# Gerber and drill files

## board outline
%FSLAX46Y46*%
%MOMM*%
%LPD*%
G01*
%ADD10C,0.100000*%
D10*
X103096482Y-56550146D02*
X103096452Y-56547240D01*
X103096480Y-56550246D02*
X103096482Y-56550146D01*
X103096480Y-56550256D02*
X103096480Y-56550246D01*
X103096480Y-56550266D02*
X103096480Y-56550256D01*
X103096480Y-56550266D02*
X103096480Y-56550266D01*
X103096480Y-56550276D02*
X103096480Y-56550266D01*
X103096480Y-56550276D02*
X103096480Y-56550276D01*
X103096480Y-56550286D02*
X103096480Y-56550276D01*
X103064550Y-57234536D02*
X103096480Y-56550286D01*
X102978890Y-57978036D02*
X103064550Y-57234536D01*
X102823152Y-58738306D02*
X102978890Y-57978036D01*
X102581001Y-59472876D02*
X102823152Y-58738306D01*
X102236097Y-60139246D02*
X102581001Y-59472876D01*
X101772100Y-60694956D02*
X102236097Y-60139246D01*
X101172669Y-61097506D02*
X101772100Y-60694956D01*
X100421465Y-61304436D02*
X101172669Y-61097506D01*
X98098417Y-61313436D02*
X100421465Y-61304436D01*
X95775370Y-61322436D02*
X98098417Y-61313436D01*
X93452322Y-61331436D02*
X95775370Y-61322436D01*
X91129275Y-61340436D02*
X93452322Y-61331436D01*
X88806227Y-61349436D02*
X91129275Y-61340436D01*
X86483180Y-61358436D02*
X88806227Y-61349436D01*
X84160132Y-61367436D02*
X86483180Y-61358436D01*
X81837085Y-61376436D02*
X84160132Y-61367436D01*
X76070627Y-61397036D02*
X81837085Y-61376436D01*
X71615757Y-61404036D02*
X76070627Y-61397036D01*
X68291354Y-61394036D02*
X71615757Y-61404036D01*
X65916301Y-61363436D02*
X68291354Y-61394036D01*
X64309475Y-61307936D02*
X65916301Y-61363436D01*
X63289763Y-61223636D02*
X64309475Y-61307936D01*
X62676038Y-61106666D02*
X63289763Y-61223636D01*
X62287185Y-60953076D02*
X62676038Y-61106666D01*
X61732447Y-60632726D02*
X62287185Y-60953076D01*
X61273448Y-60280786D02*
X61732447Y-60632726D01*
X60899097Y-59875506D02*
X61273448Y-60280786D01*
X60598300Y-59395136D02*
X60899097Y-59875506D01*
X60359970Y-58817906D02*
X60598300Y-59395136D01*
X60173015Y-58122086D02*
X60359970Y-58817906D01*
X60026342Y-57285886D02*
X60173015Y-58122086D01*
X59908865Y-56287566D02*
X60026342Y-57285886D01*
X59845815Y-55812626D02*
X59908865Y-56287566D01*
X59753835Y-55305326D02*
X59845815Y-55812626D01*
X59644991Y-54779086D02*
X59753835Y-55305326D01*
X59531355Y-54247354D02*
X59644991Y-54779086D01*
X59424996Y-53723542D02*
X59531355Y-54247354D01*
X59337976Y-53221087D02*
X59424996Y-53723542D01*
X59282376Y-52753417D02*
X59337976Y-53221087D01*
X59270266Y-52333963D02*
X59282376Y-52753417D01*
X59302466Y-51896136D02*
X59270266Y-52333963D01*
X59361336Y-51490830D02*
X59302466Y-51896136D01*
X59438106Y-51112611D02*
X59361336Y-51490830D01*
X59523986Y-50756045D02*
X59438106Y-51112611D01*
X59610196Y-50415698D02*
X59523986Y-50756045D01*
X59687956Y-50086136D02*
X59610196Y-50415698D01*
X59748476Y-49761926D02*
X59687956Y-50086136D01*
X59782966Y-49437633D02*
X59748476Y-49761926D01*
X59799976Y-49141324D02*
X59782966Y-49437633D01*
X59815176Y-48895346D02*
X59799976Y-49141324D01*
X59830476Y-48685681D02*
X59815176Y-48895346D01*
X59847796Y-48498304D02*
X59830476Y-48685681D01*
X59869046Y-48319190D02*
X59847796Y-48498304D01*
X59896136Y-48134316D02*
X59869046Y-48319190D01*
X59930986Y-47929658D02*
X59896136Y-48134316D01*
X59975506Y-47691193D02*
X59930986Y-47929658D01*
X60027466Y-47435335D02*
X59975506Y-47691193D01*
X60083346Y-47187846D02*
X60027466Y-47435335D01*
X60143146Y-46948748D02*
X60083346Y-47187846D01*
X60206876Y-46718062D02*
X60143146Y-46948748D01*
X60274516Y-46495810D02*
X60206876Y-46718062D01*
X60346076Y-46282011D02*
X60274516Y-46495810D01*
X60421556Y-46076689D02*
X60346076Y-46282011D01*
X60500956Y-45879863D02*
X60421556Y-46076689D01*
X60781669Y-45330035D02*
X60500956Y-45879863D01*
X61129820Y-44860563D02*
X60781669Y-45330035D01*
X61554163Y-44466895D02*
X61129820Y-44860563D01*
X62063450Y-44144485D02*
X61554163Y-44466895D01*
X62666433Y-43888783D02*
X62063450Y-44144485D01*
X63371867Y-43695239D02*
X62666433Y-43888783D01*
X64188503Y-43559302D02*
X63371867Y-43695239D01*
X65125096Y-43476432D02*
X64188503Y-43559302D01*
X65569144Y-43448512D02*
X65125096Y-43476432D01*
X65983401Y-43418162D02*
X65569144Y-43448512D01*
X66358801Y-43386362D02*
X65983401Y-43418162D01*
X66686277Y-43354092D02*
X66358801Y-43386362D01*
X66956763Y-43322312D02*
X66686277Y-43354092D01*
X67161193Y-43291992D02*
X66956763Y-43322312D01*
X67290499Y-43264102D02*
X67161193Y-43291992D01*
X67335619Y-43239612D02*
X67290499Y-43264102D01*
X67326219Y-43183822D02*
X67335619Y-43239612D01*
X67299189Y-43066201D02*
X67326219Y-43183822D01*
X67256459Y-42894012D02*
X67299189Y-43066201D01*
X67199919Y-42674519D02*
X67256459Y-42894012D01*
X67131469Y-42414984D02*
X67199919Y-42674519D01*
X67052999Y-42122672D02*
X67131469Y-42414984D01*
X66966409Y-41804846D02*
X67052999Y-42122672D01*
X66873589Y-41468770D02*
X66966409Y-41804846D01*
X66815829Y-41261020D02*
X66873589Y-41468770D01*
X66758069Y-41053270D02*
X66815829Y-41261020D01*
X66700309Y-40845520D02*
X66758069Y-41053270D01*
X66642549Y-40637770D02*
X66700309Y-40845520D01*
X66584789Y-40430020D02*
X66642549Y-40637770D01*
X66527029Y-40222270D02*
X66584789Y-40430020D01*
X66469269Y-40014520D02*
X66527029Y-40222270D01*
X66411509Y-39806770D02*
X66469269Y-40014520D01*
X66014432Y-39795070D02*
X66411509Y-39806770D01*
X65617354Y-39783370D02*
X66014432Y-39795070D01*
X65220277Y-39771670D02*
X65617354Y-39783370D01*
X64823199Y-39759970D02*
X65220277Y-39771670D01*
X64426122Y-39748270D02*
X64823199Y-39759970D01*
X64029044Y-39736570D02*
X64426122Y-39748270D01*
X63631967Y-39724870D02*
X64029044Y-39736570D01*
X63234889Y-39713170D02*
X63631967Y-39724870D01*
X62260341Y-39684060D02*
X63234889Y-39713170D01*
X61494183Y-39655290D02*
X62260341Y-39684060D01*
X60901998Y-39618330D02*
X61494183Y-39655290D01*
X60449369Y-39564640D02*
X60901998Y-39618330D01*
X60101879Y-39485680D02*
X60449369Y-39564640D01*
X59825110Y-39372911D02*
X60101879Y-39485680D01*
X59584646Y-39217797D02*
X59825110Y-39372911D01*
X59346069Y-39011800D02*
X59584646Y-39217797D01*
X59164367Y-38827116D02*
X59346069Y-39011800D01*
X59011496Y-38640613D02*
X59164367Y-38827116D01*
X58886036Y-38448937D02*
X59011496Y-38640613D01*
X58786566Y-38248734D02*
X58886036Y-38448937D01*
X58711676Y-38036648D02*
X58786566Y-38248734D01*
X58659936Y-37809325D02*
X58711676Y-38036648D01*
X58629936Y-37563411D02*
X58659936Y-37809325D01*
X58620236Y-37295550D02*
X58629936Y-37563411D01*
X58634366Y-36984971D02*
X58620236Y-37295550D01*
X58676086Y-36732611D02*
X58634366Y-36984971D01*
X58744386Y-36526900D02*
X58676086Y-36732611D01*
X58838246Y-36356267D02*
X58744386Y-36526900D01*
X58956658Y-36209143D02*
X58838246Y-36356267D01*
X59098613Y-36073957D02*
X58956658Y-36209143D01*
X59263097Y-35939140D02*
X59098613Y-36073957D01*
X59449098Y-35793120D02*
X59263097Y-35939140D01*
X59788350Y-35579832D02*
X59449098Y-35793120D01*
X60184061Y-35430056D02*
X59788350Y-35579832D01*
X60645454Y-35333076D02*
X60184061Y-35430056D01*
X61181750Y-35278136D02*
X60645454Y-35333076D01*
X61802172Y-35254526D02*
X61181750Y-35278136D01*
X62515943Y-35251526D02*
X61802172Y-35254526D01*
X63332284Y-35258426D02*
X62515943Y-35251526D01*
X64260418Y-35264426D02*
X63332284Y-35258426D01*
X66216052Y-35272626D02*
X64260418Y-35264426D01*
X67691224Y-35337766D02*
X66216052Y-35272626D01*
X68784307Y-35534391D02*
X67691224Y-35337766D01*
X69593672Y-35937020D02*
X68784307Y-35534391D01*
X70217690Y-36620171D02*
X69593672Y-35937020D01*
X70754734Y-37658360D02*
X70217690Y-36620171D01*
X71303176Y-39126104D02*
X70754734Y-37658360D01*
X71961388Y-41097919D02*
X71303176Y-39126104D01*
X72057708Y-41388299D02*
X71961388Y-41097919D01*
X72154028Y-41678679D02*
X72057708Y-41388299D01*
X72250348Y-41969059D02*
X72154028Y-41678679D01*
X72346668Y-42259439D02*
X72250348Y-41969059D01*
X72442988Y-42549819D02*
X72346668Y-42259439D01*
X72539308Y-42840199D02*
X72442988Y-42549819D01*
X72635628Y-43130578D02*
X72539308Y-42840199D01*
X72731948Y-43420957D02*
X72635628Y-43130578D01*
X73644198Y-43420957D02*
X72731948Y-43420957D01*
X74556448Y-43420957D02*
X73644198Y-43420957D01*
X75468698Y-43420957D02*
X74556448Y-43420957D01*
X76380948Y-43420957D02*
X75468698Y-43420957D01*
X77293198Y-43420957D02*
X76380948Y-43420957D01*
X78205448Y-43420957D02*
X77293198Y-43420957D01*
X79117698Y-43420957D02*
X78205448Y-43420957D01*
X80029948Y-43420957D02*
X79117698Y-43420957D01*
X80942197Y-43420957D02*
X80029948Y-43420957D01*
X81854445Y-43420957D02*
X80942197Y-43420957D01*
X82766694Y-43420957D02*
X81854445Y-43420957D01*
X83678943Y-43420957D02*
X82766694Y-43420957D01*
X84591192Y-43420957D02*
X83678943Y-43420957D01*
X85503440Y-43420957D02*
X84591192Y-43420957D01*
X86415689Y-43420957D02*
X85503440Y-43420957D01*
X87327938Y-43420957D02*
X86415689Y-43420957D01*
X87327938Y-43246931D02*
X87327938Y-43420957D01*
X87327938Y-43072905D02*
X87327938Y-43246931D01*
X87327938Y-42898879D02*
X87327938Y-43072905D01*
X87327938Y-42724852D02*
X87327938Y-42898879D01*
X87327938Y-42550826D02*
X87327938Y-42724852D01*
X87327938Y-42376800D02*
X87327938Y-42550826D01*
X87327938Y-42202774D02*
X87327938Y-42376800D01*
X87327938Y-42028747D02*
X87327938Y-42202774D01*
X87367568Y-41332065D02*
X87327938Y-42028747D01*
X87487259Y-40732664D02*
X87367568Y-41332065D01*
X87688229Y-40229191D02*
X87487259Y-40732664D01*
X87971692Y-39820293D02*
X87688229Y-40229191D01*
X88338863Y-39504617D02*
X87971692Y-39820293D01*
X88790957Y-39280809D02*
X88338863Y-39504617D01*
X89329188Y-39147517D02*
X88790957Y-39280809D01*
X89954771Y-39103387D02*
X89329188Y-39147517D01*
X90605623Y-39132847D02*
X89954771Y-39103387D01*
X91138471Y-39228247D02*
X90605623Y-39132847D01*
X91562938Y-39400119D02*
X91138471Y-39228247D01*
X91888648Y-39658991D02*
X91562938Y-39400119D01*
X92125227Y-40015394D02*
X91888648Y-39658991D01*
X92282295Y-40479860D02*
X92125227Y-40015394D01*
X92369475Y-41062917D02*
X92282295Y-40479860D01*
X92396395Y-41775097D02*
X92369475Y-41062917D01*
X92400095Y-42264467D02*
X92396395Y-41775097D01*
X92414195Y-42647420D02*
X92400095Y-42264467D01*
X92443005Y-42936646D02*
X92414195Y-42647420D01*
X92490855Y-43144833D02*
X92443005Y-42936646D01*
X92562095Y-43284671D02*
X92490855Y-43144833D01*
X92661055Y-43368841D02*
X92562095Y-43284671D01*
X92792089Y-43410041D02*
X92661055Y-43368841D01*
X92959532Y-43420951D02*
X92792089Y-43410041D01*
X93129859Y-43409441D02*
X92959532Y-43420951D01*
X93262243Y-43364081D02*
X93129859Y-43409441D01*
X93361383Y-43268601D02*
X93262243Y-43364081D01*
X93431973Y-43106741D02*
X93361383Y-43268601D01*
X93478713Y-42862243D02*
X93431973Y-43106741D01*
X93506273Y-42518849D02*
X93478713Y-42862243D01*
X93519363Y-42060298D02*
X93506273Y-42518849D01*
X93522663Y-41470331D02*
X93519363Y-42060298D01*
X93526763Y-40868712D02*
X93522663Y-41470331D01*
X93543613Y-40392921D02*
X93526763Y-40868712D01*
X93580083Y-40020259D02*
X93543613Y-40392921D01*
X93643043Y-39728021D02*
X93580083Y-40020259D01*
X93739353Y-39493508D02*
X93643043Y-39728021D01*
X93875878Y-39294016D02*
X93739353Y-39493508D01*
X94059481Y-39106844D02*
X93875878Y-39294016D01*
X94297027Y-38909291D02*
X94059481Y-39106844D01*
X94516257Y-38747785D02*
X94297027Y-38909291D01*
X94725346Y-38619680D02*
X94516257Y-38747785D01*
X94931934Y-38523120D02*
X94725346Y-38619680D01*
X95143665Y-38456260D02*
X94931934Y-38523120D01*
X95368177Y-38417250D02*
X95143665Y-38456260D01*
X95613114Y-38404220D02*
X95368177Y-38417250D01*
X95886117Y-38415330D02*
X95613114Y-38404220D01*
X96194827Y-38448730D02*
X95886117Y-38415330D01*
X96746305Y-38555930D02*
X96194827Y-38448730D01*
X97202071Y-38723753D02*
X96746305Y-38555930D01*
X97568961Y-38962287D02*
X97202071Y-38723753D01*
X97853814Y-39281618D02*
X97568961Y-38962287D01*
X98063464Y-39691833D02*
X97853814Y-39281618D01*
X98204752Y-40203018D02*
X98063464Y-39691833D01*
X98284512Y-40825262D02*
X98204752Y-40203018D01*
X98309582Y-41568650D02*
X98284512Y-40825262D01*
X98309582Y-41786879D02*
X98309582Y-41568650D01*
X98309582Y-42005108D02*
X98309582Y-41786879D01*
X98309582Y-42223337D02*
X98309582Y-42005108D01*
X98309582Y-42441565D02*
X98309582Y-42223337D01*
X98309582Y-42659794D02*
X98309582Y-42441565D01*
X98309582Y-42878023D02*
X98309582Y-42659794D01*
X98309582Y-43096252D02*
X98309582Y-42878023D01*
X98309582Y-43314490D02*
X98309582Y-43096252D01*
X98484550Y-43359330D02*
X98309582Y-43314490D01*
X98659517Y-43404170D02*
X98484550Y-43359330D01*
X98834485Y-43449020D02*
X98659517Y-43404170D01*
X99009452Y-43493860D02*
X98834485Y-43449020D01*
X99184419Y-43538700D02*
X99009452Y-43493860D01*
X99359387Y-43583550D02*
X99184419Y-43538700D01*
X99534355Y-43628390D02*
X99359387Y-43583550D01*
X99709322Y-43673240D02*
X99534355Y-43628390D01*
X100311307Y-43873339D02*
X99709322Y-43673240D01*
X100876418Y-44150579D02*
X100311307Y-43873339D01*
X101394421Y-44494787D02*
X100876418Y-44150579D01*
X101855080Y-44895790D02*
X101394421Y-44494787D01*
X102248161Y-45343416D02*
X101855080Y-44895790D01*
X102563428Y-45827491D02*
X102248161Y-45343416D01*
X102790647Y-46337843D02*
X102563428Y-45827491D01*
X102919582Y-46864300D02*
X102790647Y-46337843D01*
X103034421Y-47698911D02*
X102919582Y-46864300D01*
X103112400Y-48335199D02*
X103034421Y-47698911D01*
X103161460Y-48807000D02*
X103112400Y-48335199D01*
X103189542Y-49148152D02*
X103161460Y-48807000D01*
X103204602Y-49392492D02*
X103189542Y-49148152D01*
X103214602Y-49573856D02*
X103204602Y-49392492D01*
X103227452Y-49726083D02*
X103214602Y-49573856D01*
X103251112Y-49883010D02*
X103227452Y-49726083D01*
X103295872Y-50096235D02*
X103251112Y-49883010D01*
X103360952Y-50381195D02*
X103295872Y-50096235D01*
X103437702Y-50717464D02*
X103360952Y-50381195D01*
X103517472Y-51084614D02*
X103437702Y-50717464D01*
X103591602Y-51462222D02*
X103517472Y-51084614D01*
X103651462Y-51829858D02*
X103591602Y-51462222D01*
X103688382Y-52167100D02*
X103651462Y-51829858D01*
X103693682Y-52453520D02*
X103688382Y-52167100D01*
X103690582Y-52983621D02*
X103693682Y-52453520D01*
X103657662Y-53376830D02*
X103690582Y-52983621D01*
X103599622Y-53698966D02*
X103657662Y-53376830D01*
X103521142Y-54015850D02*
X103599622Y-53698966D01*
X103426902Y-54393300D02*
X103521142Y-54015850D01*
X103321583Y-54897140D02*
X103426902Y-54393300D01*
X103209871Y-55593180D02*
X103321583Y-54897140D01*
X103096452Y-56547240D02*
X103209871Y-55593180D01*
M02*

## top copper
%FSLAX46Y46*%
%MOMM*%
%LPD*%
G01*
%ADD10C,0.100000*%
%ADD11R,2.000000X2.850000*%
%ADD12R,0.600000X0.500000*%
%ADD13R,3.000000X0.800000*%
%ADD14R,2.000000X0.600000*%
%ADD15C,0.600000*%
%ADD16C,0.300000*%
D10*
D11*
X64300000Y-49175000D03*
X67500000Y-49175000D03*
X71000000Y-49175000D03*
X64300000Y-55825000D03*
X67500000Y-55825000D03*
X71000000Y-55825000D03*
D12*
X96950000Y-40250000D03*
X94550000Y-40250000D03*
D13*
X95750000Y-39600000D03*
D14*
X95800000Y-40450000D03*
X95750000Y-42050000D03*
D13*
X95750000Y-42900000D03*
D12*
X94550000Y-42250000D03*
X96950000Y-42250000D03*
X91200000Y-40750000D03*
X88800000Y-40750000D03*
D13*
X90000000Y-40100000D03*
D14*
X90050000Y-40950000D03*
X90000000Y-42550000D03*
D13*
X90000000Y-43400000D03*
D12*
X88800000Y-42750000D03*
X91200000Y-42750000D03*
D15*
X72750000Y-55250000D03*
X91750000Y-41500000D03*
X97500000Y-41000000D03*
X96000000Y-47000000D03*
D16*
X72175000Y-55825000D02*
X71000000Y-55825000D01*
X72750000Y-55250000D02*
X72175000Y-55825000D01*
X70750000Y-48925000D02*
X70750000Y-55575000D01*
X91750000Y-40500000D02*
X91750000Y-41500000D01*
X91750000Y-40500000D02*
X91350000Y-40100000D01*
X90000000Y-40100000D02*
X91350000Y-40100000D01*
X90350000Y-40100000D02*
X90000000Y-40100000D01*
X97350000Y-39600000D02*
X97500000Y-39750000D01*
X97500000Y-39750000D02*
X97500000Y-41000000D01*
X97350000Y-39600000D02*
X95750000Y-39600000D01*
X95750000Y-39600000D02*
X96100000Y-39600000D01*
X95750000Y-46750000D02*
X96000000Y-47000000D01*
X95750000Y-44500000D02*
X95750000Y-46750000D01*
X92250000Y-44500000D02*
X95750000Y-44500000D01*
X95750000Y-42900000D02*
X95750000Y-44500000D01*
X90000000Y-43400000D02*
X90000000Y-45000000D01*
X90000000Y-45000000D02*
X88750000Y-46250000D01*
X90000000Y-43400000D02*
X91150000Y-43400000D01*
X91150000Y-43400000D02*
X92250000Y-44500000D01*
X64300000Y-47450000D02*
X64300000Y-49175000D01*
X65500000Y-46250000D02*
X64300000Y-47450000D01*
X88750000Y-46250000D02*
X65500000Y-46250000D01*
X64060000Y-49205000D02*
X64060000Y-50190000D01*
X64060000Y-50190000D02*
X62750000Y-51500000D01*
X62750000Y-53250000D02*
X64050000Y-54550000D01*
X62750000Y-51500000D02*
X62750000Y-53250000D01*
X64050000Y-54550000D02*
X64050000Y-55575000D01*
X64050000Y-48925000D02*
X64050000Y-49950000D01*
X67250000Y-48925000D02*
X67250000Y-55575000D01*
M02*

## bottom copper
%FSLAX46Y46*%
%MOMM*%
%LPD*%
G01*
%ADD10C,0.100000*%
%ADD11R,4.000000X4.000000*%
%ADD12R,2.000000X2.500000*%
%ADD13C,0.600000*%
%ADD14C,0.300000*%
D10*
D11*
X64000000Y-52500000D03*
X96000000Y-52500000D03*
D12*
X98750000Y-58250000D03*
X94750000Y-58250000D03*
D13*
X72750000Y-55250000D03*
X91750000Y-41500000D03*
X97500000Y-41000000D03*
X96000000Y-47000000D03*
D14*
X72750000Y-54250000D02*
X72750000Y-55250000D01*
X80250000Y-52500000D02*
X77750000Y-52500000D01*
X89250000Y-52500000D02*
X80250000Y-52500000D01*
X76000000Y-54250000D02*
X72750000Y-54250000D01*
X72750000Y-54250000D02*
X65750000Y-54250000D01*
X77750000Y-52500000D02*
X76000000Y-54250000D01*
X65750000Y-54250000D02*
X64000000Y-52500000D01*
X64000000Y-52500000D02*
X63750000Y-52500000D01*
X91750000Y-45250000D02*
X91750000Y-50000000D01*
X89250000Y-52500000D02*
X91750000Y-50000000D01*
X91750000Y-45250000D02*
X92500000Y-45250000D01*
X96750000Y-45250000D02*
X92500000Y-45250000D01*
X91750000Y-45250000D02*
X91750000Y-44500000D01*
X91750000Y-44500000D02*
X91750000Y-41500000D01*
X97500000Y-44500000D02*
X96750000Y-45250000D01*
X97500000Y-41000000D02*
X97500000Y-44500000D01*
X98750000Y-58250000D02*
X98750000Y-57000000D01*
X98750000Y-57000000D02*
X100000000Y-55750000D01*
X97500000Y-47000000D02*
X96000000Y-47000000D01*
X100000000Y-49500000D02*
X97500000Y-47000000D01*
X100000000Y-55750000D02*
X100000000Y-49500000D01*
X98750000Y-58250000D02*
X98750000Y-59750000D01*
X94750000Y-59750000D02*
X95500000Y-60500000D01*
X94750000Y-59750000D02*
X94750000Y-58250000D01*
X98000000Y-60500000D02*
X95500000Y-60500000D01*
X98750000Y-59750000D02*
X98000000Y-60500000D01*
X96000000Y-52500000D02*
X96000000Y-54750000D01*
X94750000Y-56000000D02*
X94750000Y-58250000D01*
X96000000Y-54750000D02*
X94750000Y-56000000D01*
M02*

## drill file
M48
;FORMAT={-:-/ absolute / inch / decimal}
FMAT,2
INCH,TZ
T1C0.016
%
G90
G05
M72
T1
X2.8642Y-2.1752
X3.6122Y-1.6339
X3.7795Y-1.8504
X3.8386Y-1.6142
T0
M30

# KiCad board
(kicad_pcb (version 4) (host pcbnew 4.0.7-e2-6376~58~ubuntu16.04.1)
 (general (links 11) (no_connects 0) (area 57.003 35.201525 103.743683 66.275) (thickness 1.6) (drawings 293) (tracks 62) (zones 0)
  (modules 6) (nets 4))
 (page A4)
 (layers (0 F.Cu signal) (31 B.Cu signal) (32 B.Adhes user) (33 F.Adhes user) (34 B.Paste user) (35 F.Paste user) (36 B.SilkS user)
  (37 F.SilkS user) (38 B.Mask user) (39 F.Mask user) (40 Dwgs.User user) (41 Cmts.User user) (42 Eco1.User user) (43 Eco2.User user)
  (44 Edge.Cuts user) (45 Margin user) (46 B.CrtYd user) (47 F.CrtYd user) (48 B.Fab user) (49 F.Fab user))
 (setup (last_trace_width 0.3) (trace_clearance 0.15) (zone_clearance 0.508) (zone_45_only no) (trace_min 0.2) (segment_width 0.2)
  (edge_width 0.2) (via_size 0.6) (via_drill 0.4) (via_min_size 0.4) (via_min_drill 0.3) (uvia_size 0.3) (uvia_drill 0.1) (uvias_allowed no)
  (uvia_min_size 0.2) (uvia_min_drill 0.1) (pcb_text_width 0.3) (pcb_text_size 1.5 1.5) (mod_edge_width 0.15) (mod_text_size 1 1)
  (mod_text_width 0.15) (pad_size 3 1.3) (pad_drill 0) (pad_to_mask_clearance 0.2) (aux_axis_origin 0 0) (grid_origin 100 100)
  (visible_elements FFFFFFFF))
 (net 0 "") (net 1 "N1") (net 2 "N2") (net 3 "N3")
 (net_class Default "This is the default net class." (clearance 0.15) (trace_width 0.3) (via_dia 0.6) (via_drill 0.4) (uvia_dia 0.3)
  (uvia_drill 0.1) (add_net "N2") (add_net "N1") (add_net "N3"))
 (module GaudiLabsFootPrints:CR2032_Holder (layer B.Cu) (at 80 52.5)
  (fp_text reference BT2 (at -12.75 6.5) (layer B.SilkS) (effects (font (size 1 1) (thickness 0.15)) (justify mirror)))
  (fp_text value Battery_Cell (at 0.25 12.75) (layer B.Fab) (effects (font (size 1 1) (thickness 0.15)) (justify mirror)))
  (pad 2 smd rect (at -16 0) (size 4 4) (layers B.Cu B.Paste B.Mask) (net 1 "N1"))
  (pad 1 smd rect (at 16 0) (size 4 4) (layers B.Cu B.Paste B.Mask) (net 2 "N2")))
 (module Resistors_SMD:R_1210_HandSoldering (layer B.Cu) (at 96.75 58.25 180)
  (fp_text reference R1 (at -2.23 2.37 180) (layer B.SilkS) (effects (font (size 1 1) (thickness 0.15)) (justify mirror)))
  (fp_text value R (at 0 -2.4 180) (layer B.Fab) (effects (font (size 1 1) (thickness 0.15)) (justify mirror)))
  (pad 1 smd rect (at -2 0 180) (size 2 2.5) (layers B.Cu B.Paste B.Mask) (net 2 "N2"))
  (pad 2 smd rect (at 2 0 180) (size 2 2.5) (layers B.Cu B.Paste B.Mask) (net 2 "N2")))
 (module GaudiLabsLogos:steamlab (layer F.Cu) (at 81.14 48.34)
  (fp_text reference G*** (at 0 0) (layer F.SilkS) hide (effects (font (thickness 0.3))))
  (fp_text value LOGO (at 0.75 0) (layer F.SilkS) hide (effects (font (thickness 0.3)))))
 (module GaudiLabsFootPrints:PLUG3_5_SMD (layer F.Cu) (at 62.5 52.5 90)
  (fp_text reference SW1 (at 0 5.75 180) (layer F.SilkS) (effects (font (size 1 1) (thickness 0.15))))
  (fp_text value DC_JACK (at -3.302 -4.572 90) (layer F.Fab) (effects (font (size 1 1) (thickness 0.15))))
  (pad 1 smd rect (at 3.325 1.8 90) (size 2.85 2) (layers F.Cu F.Paste F.Mask) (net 2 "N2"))
  (pad 2 smd rect (at 3.325 5 90) (size 2.85 2) (layers F.Cu F.Paste F.Mask) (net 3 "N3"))
  (pad 3 smd rect (at 3.325 8.5 90) (size 2.85 2) (layers F.Cu F.Paste F.Mask) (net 1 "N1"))
  (pad 1 smd rect (at -3.325 1.8 90) (size 2.85 2) (layers F.Cu F.Paste F.Mask) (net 2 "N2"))
  (pad 2 smd rect (at -3.325 5 90) (size 2.85 2) (layers F.Cu F.Paste F.Mask) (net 3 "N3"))
  (pad 3 smd rect (at -3.325 8.5 90) (size 2.85 2) (layers F.Cu F.Paste F.Mask) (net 1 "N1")))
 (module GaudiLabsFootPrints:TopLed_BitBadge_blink (layer F.Cu) (at 95.75 41.25 180)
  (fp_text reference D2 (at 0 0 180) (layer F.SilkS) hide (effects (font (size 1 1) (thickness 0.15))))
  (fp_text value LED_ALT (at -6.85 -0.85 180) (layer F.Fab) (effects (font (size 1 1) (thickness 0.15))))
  (pad "" smd rect (at -1.2 1 180) (size 0.6 0.5) (layers F.Cu F.Paste F.Mask))
  (pad "" smd rect (at 1.2 1 180) (size 0.6 0.5) (layers F.Cu F.Paste F.Mask))
  (pad 1 smd rect (at 0 1.65 180) (size 3 0.8) (layers F.Cu F.Paste F.Mask) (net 1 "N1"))
  (pad "" smd rect (at -0.05 0.8 180) (size 2 0.6) (layers F.Cu F.Paste F.Mask))
  (pad "" smd rect (at 0 -0.8 180) (size 2 0.6) (layers F.Cu F.Paste F.Mask))
  (pad 2 smd rect (at 0 -1.65 180) (size 3 0.8) (layers F.Cu F.Paste F.Mask) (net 2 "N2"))
  (pad "" smd rect (at 1.2 -1 180) (size 0.6 0.5) (layers F.Cu F.Paste F.Mask))
  (pad "" smd rect (at -1.2 -1 180) (size 0.6 0.5) (layers F.Cu F.Paste F.Mask)))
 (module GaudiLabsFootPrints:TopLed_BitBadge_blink (layer F.Cu) (at 90 41.75 180)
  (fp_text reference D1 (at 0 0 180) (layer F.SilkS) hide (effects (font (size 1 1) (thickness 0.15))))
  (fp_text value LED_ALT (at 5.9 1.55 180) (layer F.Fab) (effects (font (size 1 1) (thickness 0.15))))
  (pad "" smd rect (at -1.2 1 180) (size 0.6 0.5) (layers F.Cu F.Paste F.Mask))
  (pad "" smd rect (at 1.2 1 180) (size 0.6 0.5) (layers F.Cu F.Paste F.Mask))
  (pad 1 smd rect (at 0 1.65 180) (size 3 0.8) (layers F.Cu F.Paste F.Mask) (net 1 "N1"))
  (pad "" smd rect (at -0.05 0.8 180) (size 2 0.6) (layers F.Cu F.Paste F.Mask))
  (pad "" smd rect (at 0 -0.8 180) (size 2 0.6) (layers F.Cu F.Paste F.Mask))
  (pad 2 smd rect (at 0 -1.65 180) (size 3 0.8) (layers F.Cu F.Paste F.Mask) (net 2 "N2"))
  (pad "" smd rect (at 1.2 -1 180) (size 0.6 0.5) (layers F.Cu F.Paste F.Mask))
  (pad "" smd rect (at -1.2 -1 180) (size 0.6 0.5) (layers F.Cu F.Paste F.Mask)))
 (gr_line (start 103.096482 56.550146) (end 103.096452 56.54724) (layer Edge.Cuts) (width 0.1))
 (gr_line (start 103.09648 56.550246) (end 103.096482 56.550146) (layer Edge.Cuts) (width 0.1))
 (gr_line (start 103.09648 56.550256) (end 103.09648 56.550246) (layer Edge.Cuts) (width 0.1))
 (gr_line (start 103.09648 56.550266) (end 103.09648 56.550256) (layer Edge.Cuts) (width 0.1))
 (gr_line (start 103.09648 56.550266) (end 103.09648 56.550266) (layer Edge.Cuts) (width 0.1))
 (gr_line (start 103.09648 56.550276) (end 103.09648 56.550266) (layer Edge.Cuts) (width 0.1))
 (gr_line (start 103.09648 56.550276) (end 103.09648 56.550276) (layer Edge.Cuts) (width 0.1))
 (gr_line (start 103.09648 56.550286) (end 103.09648 56.550276) (layer Edge.Cuts) (width 0.1))
 (gr_line (start 103.06455 57.234536) (end 103.09648 56.550286) (layer Edge.Cuts) (width 0.1))
 (gr_line (start 102.97889 57.978036) (end 103.06455 57.234536) (layer Edge.Cuts) (width 0.1))
 (gr_line (start 102.823152 58.738306) (end 102.97889 57.978036) (layer Edge.Cuts) (width 0.1))
 (gr_line (start 102.581001 59.472876) (end 102.823152 58.738306) (layer Edge.Cuts) (width 0.1))
 (gr_line (start 102.236097 60.139246) (end 102.581001 59.472876) (layer Edge.Cuts) (width 0.1))
 (gr_line (start 101.7721 60.694956) (end 102.236097 60.139246) (layer Edge.Cuts) (width 0.1))
 (gr_line (start 101.172669 61.097506) (end 101.7721 60.694956) (layer Edge.Cuts) (width 0.1))
 (gr_line (start 100.421465 61.304436) (end 101.172669 61.097506) (layer Edge.Cuts) (width 0.1))
 (gr_line (start 98.098417 61.313436) (end 100.421465 61.304436) (layer Edge.Cuts) (width 0.1))
 (gr_line (start 95.77537 61.322436) (end 98.098417 61.313436) (layer Edge.Cuts) (width 0.1))
 (gr_line (start 93.452322 61.331436) (end 95.77537 61.322436) (layer Edge.Cuts) (width 0.1))
 (gr_line (start 91.129275 61.340436) (end 93.452322 61.331436) (layer Edge.Cuts) (width 0.1))
 (gr_line (start 88.806227 61.349436) (end 91.129275 61.340436) (layer Edge.Cuts) (width 0.1))
 (gr_line (start 86.48318 61.358436) (end 88.806227 61.349436) (layer Edge.Cuts) (width 0.1))
 (gr_line (start 84.160132 61.367436) (end 86.48318 61.358436) (layer Edge.Cuts) (width 0.1))
 (gr_line (start 81.837085 61.376436) (end 84.160132 61.367436) (layer Edge.Cuts) (width 0.1))
 (gr_line (start 76.070627 61.397036) (end 81.837085 61.376436) (layer Edge.Cuts) (width 0.1))
 (gr_line (start 71.615757 61.404036) (end 76.070627 61.397036) (layer Edge.Cuts) (width 0.1))
 (gr_line (start 68.291354 61.394036) (end 71.615757 61.404036) (layer Edge.Cuts) (width 0.1))
 (gr_line (start 65.916301 61.363436) (end 68.291354 61.394036) (layer Edge.Cuts) (width 0.1))
 (gr_line (start 64.309475 61.307936) (end 65.916301 61.363436) (layer Edge.Cuts) (width 0.1))
 (gr_line (start 63.289763 61.223636) (end 64.309475 61.307936) (layer Edge.Cuts) (width 0.1))
 (gr_line (start 62.676038 61.106666) (end 63.289763 61.223636) (layer Edge.Cuts) (width 0.1))
 (gr_line (start 62.287185 60.953076) (end 62.676038 61.106666) (layer Edge.Cuts) (width 0.1))
 (gr_line (start 61.732447 60.632726) (end 62.287185 60.953076) (layer Edge.Cuts) (width 0.1))
 (gr_line (start 61.273448 60.280786) (end 61.732447 60.632726) (layer Edge.Cuts) (width 0.1))
 (gr_line (start 60.899097 59.875506) (end 61.273448 60.280786) (layer Edge.Cuts) (width 0.1))
 (gr_line (start 60.5983 59.395136) (end 60.899097 59.875506) (layer Edge.Cuts) (width 0.1))
 (gr_line (start 60.35997 58.817906) (end 60.5983 59.395136) (layer Edge.Cuts) (width 0.1))
 (gr_line (start 60.173015 58.122086) (end 60.35997 58.817906) (layer Edge.Cuts) (width 0.1))
 (gr_line (start 60.026342 57.285886) (end 60.173015 58.122086) (layer Edge.Cuts) (width 0.1))
 (gr_line (start 59.908865 56.287566) (end 60.026342 57.285886) (layer Edge.Cuts) (width 0.1))
 (gr_line (start 59.845815 55.812626) (end 59.908865 56.287566) (layer Edge.Cuts) (width 0.1))
 (gr_line (start 59.753835 55.305326) (end 59.845815 55.812626) (layer Edge.Cuts) (width 0.1))
 (gr_line (start 59.644991 54.779086) (end 59.753835 55.305326) (layer Edge.Cuts) (width 0.1))
 (gr_line (start 59.531355 54.247354) (end 59.644991 54.779086) (layer Edge.Cuts) (width 0.1))
 (gr_line (start 59.424996 53.723542) (end 59.531355 54.247354) (layer Edge.Cuts) (width 0.1))
 (gr_line (start 59.337976 53.221087) (end 59.424996 53.723542) (layer Edge.Cuts) (width 0.1))
 (gr_line (start 59.282376 52.753417) (end 59.337976 53.221087) (layer Edge.Cuts) (width 0.1))
 (gr_line (start 59.270266 52.333963) (end 59.282376 52.753417) (layer Edge.Cuts) (width 0.1))
 (gr_line (start 59.302466 51.896136) (end 59.270266 52.333963) (layer Edge.Cuts) (width 0.1))
 (gr_line (start 59.361336 51.49083) (end 59.302466 51.896136) (layer Edge.Cuts) (width 0.1))
 (gr_line (start 59.438106 51.112611) (end 59.361336 51.49083) (layer Edge.Cuts) (width 0.1))
 (gr_line (start 59.523986 50.756045) (end 59.438106 51.112611) (layer Edge.Cuts) (width 0.1))
 (gr_line (start 59.610196 50.415698) (end 59.523986 50.756045) (layer Edge.Cuts) (width 0.1))
 (gr_line (start 59.687956 50.086136) (end 59.610196 50.415698) (layer Edge.Cuts) (width 0.1))
 (gr_line (start 59.748476 49.761926) (end 59.687956 50.086136) (layer Edge.Cuts) (width 0.1))
 (gr_line (start 59.782966 49.437633) (end 59.748476 49.761926) (layer Edge.Cuts) (width 0.1))
 (gr_line (start 59.799976 49.141324) (end 59.782966 49.437633) (layer Edge.Cuts) (width 0.1))
 (gr_line (start 59.815176 48.895346) (end 59.799976 49.141324) (layer Edge.Cuts) (width 0.1))
 (gr_line (start 59.830476 48.685681) (end 59.815176 48.895346) (layer Edge.Cuts) (width 0.1))
 (gr_line (start 59.847796 48.498304) (end 59.830476 48.685681) (layer Edge.Cuts) (width 0.1))
 (gr_line (start 59.869046 48.31919) (end 59.847796 48.498304) (layer Edge.Cuts) (width 0.1))
 (gr_line (start 59.896136 48.134316) (end 59.869046 48.31919) (layer Edge.Cuts) (width 0.1))
 (gr_line (start 59.930986 47.929658) (end 59.896136 48.134316) (layer Edge.Cuts) (width 0.1))
 (gr_line (start 59.975506 47.691193) (end 59.930986 47.929658) (layer Edge.Cuts) (width 0.1))
 (gr_line (start 60.027466 47.435335) (end 59.975506 47.691193) (layer Edge.Cuts) (width 0.1))
 (gr_line (start 60.083346 47.187846) (end 60.027466 47.435335) (layer Edge.Cuts) (width 0.1))
 (gr_line (start 60.143146 46.948748) (end 60.083346 47.187846) (layer Edge.Cuts) (width 0.1))
 (gr_line (start 60.206876 46.718062) (end 60.143146 46.948748) (layer Edge.Cuts) (width 0.1))
 (gr_line (start 60.274516 46.49581) (end 60.206876 46.718062) (layer Edge.Cuts) (width 0.1))
 (gr_line (start 60.346076 46.282011) (end 60.274516 46.49581) (layer Edge.Cuts) (width 0.1))
 (gr_line (start 60.421556 46.076689) (end 60.346076 46.282011) (layer Edge.Cuts) (width 0.1))
 (gr_line (start 60.500956 45.879863) (end 60.421556 46.076689) (layer Edge.Cuts) (width 0.1))
 (gr_line (start 60.781669 45.330035) (end 60.500956 45.879863) (layer Edge.Cuts) (width 0.1))
 (gr_line (start 61.12982 44.860563) (end 60.781669 45.330035) (layer Edge.Cuts) (width 0.1))
 (gr_line (start 61.554163 44.466895) (end 61.12982 44.860563) (layer Edge.Cuts) (width 0.1))
 (gr_line (start 62.06345 44.144485) (end 61.554163 44.466895) (layer Edge.Cuts) (width 0.1))
 (gr_line (start 62.666433 43.888783) (end 62.06345 44.144485) (layer Edge.Cuts) (width 0.1))
 (gr_line (start 63.371867 43.695239) (end 62.666433 43.888783) (layer Edge.Cuts) (width 0.1))
 (gr_line (start 64.188503 43.559302) (end 63.371867 43.695239) (layer Edge.Cuts) (width 0.1))
 (gr_line (start 65.125096 43.476432) (end 64.188503 43.559302) (layer Edge.Cuts) (width 0.1))
 (gr_line (start 65.569144 43.448512) (end 65.125096 43.476432) (layer Edge.Cuts) (width 0.1))
 (gr_line (start 65.983401 43.418162) (end 65.569144 43.448512) (layer Edge.Cuts) (width 0.1))
 (gr_line (start 66.358801 43.386362) (end 65.983401 43.418162) (layer Edge.Cuts) (width 0.1))
 (gr_line (start 66.686277 43.354092) (end 66.358801 43.386362) (layer Edge.Cuts) (width 0.1))
 (gr_line (start 66.956763 43.322312) (end 66.686277 43.354092) (layer Edge.Cuts) (width 0.1))
 (gr_line (start 67.161193 43.291992) (end 66.956763 43.322312) (layer Edge.Cuts) (width 0.1))
 (gr_line (start 67.290499 43.264102) (end 67.161193 43.291992) (layer Edge.Cuts) (width 0.1))
 (gr_line (start 67.335619 43.239612) (end 67.290499 43.264102) (layer Edge.Cuts) (width 0.1))
 (gr_line (start 67.326219 43.183822) (end 67.335619 43.239612) (layer Edge.Cuts) (width 0.1))
 (gr_line (start 67.299189 43.066201) (end 67.326219 43.183822) (layer Edge.Cuts) (width 0.1))
 (gr_line (start 67.256459 42.894012) (end 67.299189 43.066201) (layer Edge.Cuts) (width 0.1))
 (gr_line (start 67.199919 42.674519) (end 67.256459 42.894012) (layer Edge.Cuts) (width 0.1))
 (gr_line (start 67.131469 42.414984) (end 67.199919 42.674519) (layer Edge.Cuts) (width 0.1))
 (gr_line (start 67.052999 42.122672) (end 67.131469 42.414984) (layer Edge.Cuts) (width 0.1))
 (gr_line (start 66.966409 41.804846) (end 67.052999 42.122672) (layer Edge.Cuts) (width 0.1))
 (gr_line (start 66.873589 41.46877) (end 66.966409 41.804846) (layer Edge.Cuts) (width 0.1))
 (gr_line (start 66.815829 41.26102) (end 66.873589 41.46877) (layer Edge.Cuts) (width 0.1))
 (gr_line (start 66.758069 41.05327) (end 66.815829 41.26102) (layer Edge.Cuts) (width 0.1))
 (gr_line (start 66.700309 40.84552) (end 66.758069 41.05327) (layer Edge.Cuts) (width 0.1))
 (gr_line (start 66.642549 40.63777) (end 66.700309 40.84552) (layer Edge.Cuts) (width 0.1))
 (gr_line (start 66.584789 40.43002) (end 66.642549 40.63777) (layer Edge.Cuts) (width 0.1))
 (gr_line (start 66.527029 40.22227) (end 66.584789 40.43002) (layer Edge.Cuts) (width 0.1))
 (gr_line (start 66.469269 40.01452) (end 66.527029 40.22227) (layer Edge.Cuts) (width 0.1))
 (gr_line (start 66.411509 39.80677) (end 66.469269 40.01452) (layer Edge.Cuts) (width 0.1))
 (gr_line (start 66.014432 39.79507) (end 66.411509 39.80677) (layer Edge.Cuts) (width 0.1))
 (gr_line (start 65.617354 39.78337) (end 66.014432 39.79507) (layer Edge.Cuts) (width 0.1))
 (gr_line (start 65.220277 39.77167) (end 65.617354 39.78337) (layer Edge.Cuts) (width 0.1))
 (gr_line (start 64.823199 39.75997) (end 65.220277 39.77167) (layer Edge.Cuts) (width 0.1))
 (gr_line (start 64.426122 39.74827) (end 64.823199 39.75997) (layer Edge.Cuts) (width 0.1))
 (gr_line (start 64.029044 39.73657) (end 64.426122 39.74827) (layer Edge.Cuts) (width 0.1))
 (gr_line (start 63.631967 39.72487) (end 64.029044 39.73657) (layer Edge.Cuts) (width 0.1))
 (gr_line (start 63.234889 39.71317) (end 63.631967 39.72487) (layer Edge.Cuts) (width 0.1))
 (gr_line (start 62.260341 39.68406) (end 63.234889 39.71317) (layer Edge.Cuts) (width 0.1))
 (gr_line (start 61.494183 39.65529) (end 62.260341 39.68406) (layer Edge.Cuts) (width 0.1))
 (gr_line (start 60.901998 39.61833) (end 61.494183 39.65529) (layer Edge.Cuts) (width 0.1))
 (gr_line (start 60.449369 39.56464) (end 60.901998 39.61833) (layer Edge.Cuts) (width 0.1))
 (gr_line (start 60.101879 39.48568) (end 60.449369 39.56464) (layer Edge.Cuts) (width 0.1))
 (gr_line (start 59.82511 39.372911) (end 60.101879 39.48568) (layer Edge.Cuts) (width 0.1))
 (gr_line (start 59.584646 39.217797) (end 59.82511 39.372911) (layer Edge.Cuts) (width 0.1))
 (gr_line (start 59.346069 39.0118) (end 59.584646 39.217797) (layer Edge.Cuts) (width 0.1))
 (gr_line (start 59.164367 38.827116) (end 59.346069 39.0118) (layer Edge.Cuts) (width 0.1))
 (gr_line (start 59.011496 38.640613) (end 59.164367 38.827116) (layer Edge.Cuts) (width 0.1))
 (gr_line (start 58.886036 38.448937) (end 59.011496 38.640613) (layer Edge.Cuts) (width 0.1))
 (gr_line (start 58.786566 38.248734) (end 58.886036 38.448937) (layer Edge.Cuts) (width 0.1))
 (gr_line (start 58.711676 38.036648) (end 58.786566 38.248734) (layer Edge.Cuts) (width 0.1))
 (gr_line (start 58.659936 37.809325) (end 58.711676 38.036648) (layer Edge.Cuts) (width 0.1))
 (gr_line (start 58.629936 37.563411) (end 58.659936 37.809325) (layer Edge.Cuts) (width 0.1))
 (gr_line (start 58.620236 37.29555) (end 58.629936 37.563411) (layer Edge.Cuts) (width 0.1))
 (gr_line (start 58.634366 36.984971) (end 58.620236 37.29555) (layer Edge.Cuts) (width 0.1))
 (gr_line (start 58.676086 36.732611) (end 58.634366 36.984971) (layer Edge.Cuts) (width 0.1))
 (gr_line (start 58.744386 36.5269) (end 58.676086 36.732611) (layer Edge.Cuts) (width 0.1))
 (gr_line (start 58.838246 36.356267) (end 58.744386 36.5269) (layer Edge.Cuts) (width 0.1))
 (gr_line (start 58.956658 36.209143) (end 58.838246 36.356267) (layer Edge.Cuts) (width 0.1))
 (gr_line (start 59.098613 36.073957) (end 58.956658 36.209143) (layer Edge.Cuts) (width 0.1))
 (gr_line (start 59.263097 35.93914) (end 59.098613 36.073957) (layer Edge.Cuts) (width 0.1))
 (gr_line (start 59.449098 35.79312) (end 59.263097 35.93914) (layer Edge.Cuts) (width 0.1))
 (gr_line (start 59.78835 35.579832) (end 59.449098 35.79312) (layer Edge.Cuts) (width 0.1))
 (gr_line (start 60.184061 35.430056) (end 59.78835 35.579832) (layer Edge.Cuts) (width 0.1))
 (gr_line (start 60.645454 35.333076) (end 60.184061 35.430056) (layer Edge.Cuts) (width 0.1))
 (gr_line (start 61.18175 35.278136) (end 60.645454 35.333076) (layer Edge.Cuts) (width 0.1))
 (gr_line (start 61.802172 35.254526) (end 61.18175 35.278136) (layer Edge.Cuts) (width 0.1))
 (gr_line (start 62.515943 35.251526) (end 61.802172 35.254526) (layer Edge.Cuts) (width 0.1))
 (gr_line (start 63.332284 35.258426) (end 62.515943 35.251526) (layer Edge.Cuts) (width 0.1))
 (gr_line (start 64.260418 35.264426) (end 63.332284 35.258426) (layer Edge.Cuts) (width 0.1))
 (gr_line (start 66.216052 35.272626) (end 64.260418 35.264426) (layer Edge.Cuts) (width 0.1))
 (gr_line (start 67.691224 35.337766) (end 66.216052 35.272626) (layer Edge.Cuts) (width 0.1))
 (gr_line (start 68.784307 35.534391) (end 67.691224 35.337766) (layer Edge.Cuts) (width 0.1))
 (gr_line (start 69.593672 35.93702) (end 68.784307 35.534391) (layer Edge.Cuts) (width 0.1))
 (gr_line (start 70.21769 36.620171) (end 69.593672 35.93702) (layer Edge.Cuts) (width 0.1))
 (gr_line (start 70.754734 37.65836) (end 70.21769 36.620171) (layer Edge.Cuts) (width 0.1))
 (gr_line (start 71.303176 39.126104) (end 70.754734 37.65836) (layer Edge.Cuts) (width 0.1))
 (gr_line (start 71.961388 41.097919) (end 71.303176 39.126104) (layer Edge.Cuts) (width 0.1))
 (gr_line (start 72.057708 41.388299) (end 71.961388 41.097919) (layer Edge.Cuts) (width 0.1))
 (gr_line (start 72.154028 41.678679) (end 72.057708 41.388299) (layer Edge.Cuts) (width 0.1))
 (gr_line (start 72.250348 41.969059) (end 72.154028 41.678679) (layer Edge.Cuts) (width 0.1))
 (gr_line (start 72.346668 42.259439) (end 72.250348 41.969059) (layer Edge.Cuts) (width 0.1))
 (gr_line (start 72.442988 42.549819) (end 72.346668 42.259439) (layer Edge.Cuts) (width 0.1))
 (gr_line (start 72.539308 42.840199) (end 72.442988 42.549819) (layer Edge.Cuts) (width 0.1))
 (gr_line (start 72.635628 43.130578) (end 72.539308 42.840199) (layer Edge.Cuts) (width 0.1))
 (gr_line (start 72.731948 43.420957) (end 72.635628 43.130578) (layer Edge.Cuts) (width 0.1))
 (gr_line (start 73.644198 43.420957) (end 72.731948 43.420957) (layer Edge.Cuts) (width 0.1))
 (gr_line (start 74.556448 43.420957) (end 73.644198 43.420957) (layer Edge.Cuts) (width 0.1))
 (gr_line (start 75.468698 43.420957) (end 74.556448 43.420957) (layer Edge.Cuts) (width 0.1))
 (gr_line (start 76.380948 43.420957) (end 75.468698 43.420957) (layer Edge.Cuts) (width 0.1))
 (gr_line (start 77.293198 43.420957) (end 76.380948 43.420957) (layer Edge.Cuts) (width 0.1))
 (gr_line (start 78.205448 43.420957) (end 77.293198 43.420957) (layer Edge.Cuts) (width 0.1))
 (gr_line (start 79.117698 43.420957) (end 78.205448 43.420957) (layer Edge.Cuts) (width 0.1))
 (gr_line (start 80.029948 43.420957) (end 79.117698 43.420957) (layer Edge.Cuts) (width 0.1))
 (gr_line (start 80.942197 43.420957) (end 80.029948 43.420957) (layer Edge.Cuts) (width 0.1))
 (gr_line (start 81.854445 43.420957) (end 80.942197 43.420957) (layer Edge.Cuts) (width 0.1))
 (gr_line (start 82.766694 43.420957) (end 81.854445 43.420957) (layer Edge.Cuts) (width 0.1))
 (gr_line (start 83.678943 43.420957) (end 82.766694 43.420957) (layer Edge.Cuts) (width 0.1))
 (gr_line (start 84.591192 43.420957) (end 83.678943 43.420957) (layer Edge.Cuts) (width 0.1))
 (gr_line (start 85.50344 43.420957) (end 84.591192 43.420957) (layer Edge.Cuts) (width 0.1))
 (gr_line (start 86.415689 43.420957) (end 85.50344 43.420957) (layer Edge.Cuts) (width 0.1))
 (gr_line (start 87.327938 43.420957) (end 86.415689 43.420957) (layer Edge.Cuts) (width 0.1))
 (gr_line (start 87.327938 43.246931) (end 87.327938 43.420957) (layer Edge.Cuts) (width 0.1))
 (gr_line (start 87.327938 43.072905) (end 87.327938 43.246931) (layer Edge.Cuts) (width 0.1))
 (gr_line (start 87.327938 42.898879) (end 87.327938 43.072905) (layer Edge.Cuts) (width 0.1))
 (gr_line (start 87.327938 42.724852) (end 87.327938 42.898879) (layer Edge.Cuts) (width 0.1))
 (gr_line (start 87.327938 42.550826) (end 87.327938 42.724852) (layer Edge.Cuts) (width 0.1))
 (gr_line (start 87.327938 42.3768) (end 87.327938 42.550826) (layer Edge.Cuts) (width 0.1))
 (gr_line (start 87.327938 42.202774) (end 87.327938 42.3768) (layer Edge.Cuts) (width 0.1))
 (gr_line (start 87.327938 42.028747) (end 87.327938 42.202774) (layer Edge.Cuts) (width 0.1))
 (gr_line (start 87.367568 41.332065) (end 87.327938 42.028747) (layer Edge.Cuts) (width 0.1))
 (gr_line (start 87.487259 40.732664) (end 87.367568 41.332065) (layer Edge.Cuts) (width 0.1))
 (gr_line (start 87.688229 40.229191) (end 87.487259 40.732664) (layer Edge.Cuts) (width 0.1))
 (gr_line (start 87.971692 39.820293) (end 87.688229 40.229191) (layer Edge.Cuts) (width 0.1))
 (gr_line (start 88.338863 39.504617) (end 87.971692 39.820293) (layer Edge.Cuts) (width 0.1))
 (gr_line (start 88.790957 39.280809) (end 88.338863 39.504617) (layer Edge.Cuts) (width 0.1))
 (gr_line (start 89.329188 39.147517) (end 88.790957 39.280809) (layer Edge.Cuts) (width 0.1))
 (gr_line (start 89.954771 39.103387) (end 89.329188 39.147517) (layer Edge.Cuts) (width 0.1))
 (gr_line (start 90.605623 39.132847) (end 89.954771 39.103387) (layer Edge.Cuts) (width 0.1))
 (gr_line (start 91.138471 39.228247) (end 90.605623 39.132847) (layer Edge.Cuts) (width 0.1))
 (gr_line (start 91.562938 39.400119) (end 91.138471 39.228247) (layer Edge.Cuts) (width 0.1))
 (gr_line (start 91.888648 39.658991) (end 91.562938 39.400119) (layer Edge.Cuts) (width 0.1))
 (gr_line (start 92.125227 40.015394) (end 91.888648 39.658991) (layer Edge.Cuts) (width 0.1))
 (gr_line (start 92.282295 40.47986) (end 92.125227 40.015394) (layer Edge.Cuts) (width 0.1))
 (gr_line (start 92.369475 41.062917) (end 92.282295 40.47986) (layer Edge.Cuts) (width 0.1))
 (gr_line (start 92.396395 41.775097) (end 92.369475 41.062917) (layer Edge.Cuts) (width 0.1))
 (gr_line (start 92.400095 42.264467) (end 92.396395 41.775097) (layer Edge.Cuts) (width 0.1))
 (gr_line (start 92.414195 42.64742) (end 92.400095 42.264467) (layer Edge.Cuts) (width 0.1))
 (gr_line (start 92.443005 42.936646) (end 92.414195 42.64742) (layer Edge.Cuts) (width 0.1))
 (gr_line (start 92.490855 43.144833) (end 92.443005 42.936646) (layer Edge.Cuts) (width 0.1))
 (gr_line (start 92.562095 43.284671) (end 92.490855 43.144833) (layer Edge.Cuts) (width 0.1))
 (gr_line (start 92.661055 43.368841) (end 92.562095 43.284671) (layer Edge.Cuts) (width 0.1))
 (gr_line (start 92.792089 43.410041) (end 92.661055 43.368841) (layer Edge.Cuts) (width 0.1))
 (gr_line (start 92.959532 43.420951) (end 92.792089 43.410041) (layer Edge.Cuts) (width 0.1))
 (gr_line (start 93.129859 43.409441) (end 92.959532 43.420951) (layer Edge.Cuts) (width 0.1))
 (gr_line (start 93.262243 43.364081) (end 93.129859 43.409441) (layer Edge.Cuts) (width 0.1))
 (gr_line (start 93.361383 43.268601) (end 93.262243 43.364081) (layer Edge.Cuts) (width 0.1))
 (gr_line (start 93.431973 43.106741) (end 93.361383 43.268601) (layer Edge.Cuts) (width 0.1))
 (gr_line (start 93.478713 42.862243) (end 93.431973 43.106741) (layer Edge.Cuts) (width 0.1))
 (gr_line (start 93.506273 42.518849) (end 93.478713 42.862243) (layer Edge.Cuts) (width 0.1))
 (gr_line (start 93.519363 42.060298) (end 93.506273 42.518849) (layer Edge.Cuts) (width 0.1))
 (gr_line (start 93.522663 41.470331) (end 93.519363 42.060298) (layer Edge.Cuts) (width 0.1))
 (gr_line (start 93.526763 40.868712) (end 93.522663 41.470331) (layer Edge.Cuts) (width 0.1))
 (gr_line (start 93.543613 40.392921) (end 93.526763 40.868712) (layer Edge.Cuts) (width 0.1))
 (gr_line (start 93.580083 40.020259) (end 93.543613 40.392921) (layer Edge.Cuts) (width 0.1))
 (gr_line (start 93.643043 39.728021) (end 93.580083 40.020259) (layer Edge.Cuts) (width 0.1))
 (gr_line (start 93.739353 39.493508) (end 93.643043 39.728021) (layer Edge.Cuts) (width 0.1))
 (gr_line (start 93.875878 39.294016) (end 93.739353 39.493508) (layer Edge.Cuts) (width 0.1))
 (gr_line (start 94.059481 39.106844) (end 93.875878 39.294016) (layer Edge.Cuts) (width 0.1))
 (gr_line (start 94.297027 38.909291) (end 94.059481 39.106844) (layer Edge.Cuts) (width 0.1))
 (gr_line (start 94.516257 38.747785) (end 94.297027 38.909291) (layer Edge.Cuts) (width 0.1))
 (gr_line (start 94.725346 38.61968) (end 94.516257 38.747785) (layer Edge.Cuts) (width 0.1))
 (gr_line (start 94.931934 38.52312) (end 94.725346 38.61968) (layer Edge.Cuts) (width 0.1))
 (gr_line (start 95.143665 38.45626) (end 94.931934 38.52312) (layer Edge.Cuts) (width 0.1))
 (gr_line (start 95.368177 38.41725) (end 95.143665 38.45626) (layer Edge.Cuts) (width 0.1))
 (gr_line (start 95.613114 38.40422) (end 95.368177 38.41725) (layer Edge.Cuts) (width 0.1))
 (gr_line (start 95.886117 38.41533) (end 95.613114 38.40422) (layer Edge.Cuts) (width 0.1))
 (gr_line (start 96.194827 38.44873) (end 95.886117 38.41533) (layer Edge.Cuts) (width 0.1))
 (gr_line (start 96.746305 38.55593) (end 96.194827 38.44873) (layer Edge.Cuts) (width 0.1))
 (gr_line (start 97.202071 38.723753) (end 96.746305 38.55593) (layer Edge.Cuts) (width 0.1))
 (gr_line (start 97.568961 38.962287) (end 97.202071 38.723753) (layer Edge.Cuts) (width 0.1))
 (gr_line (start 97.853814 39.281618) (end 97.568961 38.962287) (layer Edge.Cuts) (width 0.1))
 (gr_line (start 98.063464 39.691833) (end 97.853814 39.281618) (layer Edge.Cuts) (width 0.1))
 (gr_line (start 98.204752 40.203018) (end 98.063464 39.691833) (layer Edge.Cuts) (width 0.1))
 (gr_line (start 98.284512 40.825262) (end 98.204752 40.203018) (layer Edge.Cuts) (width 0.1))
 (gr_line (start 98.309582 41.56865) (end 98.284512 40.825262) (layer Edge.Cuts) (width 0.1))
 (gr_line (start 98.309582 41.786879) (end 98.309582 41.56865) (layer Edge.Cuts) (width 0.1))
 (gr_line (start 98.309582 42.005108) (end 98.309582 41.786879) (layer Edge.Cuts) (width 0.1))
 (gr_line (start 98.309582 42.223337) (end 98.309582 42.005108) (layer Edge.Cuts) (width 0.1))
 (gr_line (start 98.309582 42.441565) (end 98.309582 42.223337) (layer Edge.Cuts) (width 0.1))
 (gr_line (start 98.309582 42.659794) (end 98.309582 42.441565) (layer Edge.Cuts) (width 0.1))
 (gr_line (start 98.309582 42.878023) (end 98.309582 42.659794) (layer Edge.Cuts) (width 0.1))
 (gr_line (start 98.309582 43.096252) (end 98.309582 42.878023) (layer Edge.Cuts) (width 0.1))
 (gr_line (start 98.309582 43.31449) (end 98.309582 43.096252) (layer Edge.Cuts) (width 0.1))
 (gr_line (start 98.48455 43.35933) (end 98.309582 43.31449) (layer Edge.Cuts) (width 0.1))
 (gr_line (start 98.659517 43.40417) (end 98.48455 43.35933) (layer Edge.Cuts) (width 0.1))
 (gr_line (start 98.834485 43.44902) (end 98.659517 43.40417) (layer Edge.Cuts) (width 0.1))
 (gr_line (start 99.009452 43.49386) (end 98.834485 43.44902) (layer Edge.Cuts) (width 0.1))
 (gr_line (start 99.184419 43.5387) (end 99.009452 43.49386) (layer Edge.Cuts) (width 0.1))
 (gr_line (start 99.359387 43.58355) (end 99.184419 43.5387) (layer Edge.Cuts) (width 0.1))
 (gr_line (start 99.534355 43.62839) (end 99.359387 43.58355) (layer Edge.Cuts) (width 0.1))
 (gr_line (start 99.709322 43.67324) (end 99.534355 43.62839) (layer Edge.Cuts) (width 0.1))
 (gr_line (start 100.311307 43.873339) (end 99.709322 43.67324) (layer Edge.Cuts) (width 0.1))
 (gr_line (start 100.876418 44.150579) (end 100.311307 43.873339) (layer Edge.Cuts) (width 0.1))
 (gr_line (start 101.394421 44.494787) (end 100.876418 44.150579) (layer Edge.Cuts) (width 0.1))
 (gr_line (start 101.85508 44.89579) (end 101.394421 44.494787) (layer Edge.Cuts) (width 0.1))
 (gr_line (start 102.248161 45.343416) (end 101.85508 44.89579) (layer Edge.Cuts) (width 0.1))
 (gr_line (start 102.563428 45.827491) (end 102.248161 45.343416) (layer Edge.Cuts) (width 0.1))
 (gr_line (start 102.790647 46.337843) (end 102.563428 45.827491) (layer Edge.Cuts) (width 0.1))
 (gr_line (start 102.919582 46.8643) (end 102.790647 46.337843) (layer Edge.Cuts) (width 0.1))
 (gr_line (start 103.034421 47.698911) (end 102.919582 46.8643) (layer Edge.Cuts) (width 0.1))
 (gr_line (start 103.1124 48.335199) (end 103.034421 47.698911) (layer Edge.Cuts) (width 0.1))
 (gr_line (start 103.16146 48.807) (end 103.1124 48.335199) (layer Edge.Cuts) (width 0.1))
 (gr_line (start 103.189542 49.148152) (end 103.16146 48.807) (layer Edge.Cuts) (width 0.1))
 (gr_line (start 103.204602 49.392492) (end 103.189542 49.148152) (layer Edge.Cuts) (width 0.1))
 (gr_line (start 103.214602 49.573856) (end 103.204602 49.392492) (layer Edge.Cuts) (width 0.1))
 (gr_line (start 103.227452 49.726083) (end 103.214602 49.573856) (layer Edge.Cuts) (width 0.1))
 (gr_line (start 103.251112 49.88301) (end 103.227452 49.726083) (layer Edge.Cuts) (width 0.1))
 (gr_line (start 103.295872 50.096235) (end 103.251112 49.88301) (layer Edge.Cuts) (width 0.1))
 (gr_line (start 103.360952 50.381195) (end 103.295872 50.096235) (layer Edge.Cuts) (width 0.1))
 (gr_line (start 103.437702 50.717464) (end 103.360952 50.381195) (layer Edge.Cuts) (width 0.1))
 (gr_line (start 103.517472 51.084614) (end 103.437702 50.717464) (layer Edge.Cuts) (width 0.1))
 (gr_line (start 103.591602 51.462222) (end 103.517472 51.084614) (layer Edge.Cuts) (width 0.1))
 (gr_line (start 103.651462 51.829858) (end 103.591602 51.462222) (layer Edge.Cuts) (width 0.1))
 (gr_line (start 103.688382 52.1671) (end 103.651462 51.829858) (layer Edge.Cuts) (width 0.1))
 (gr_line (start 103.693682 52.45352) (end 103.688382 52.1671) (layer Edge.Cuts) (width 0.1))
 (gr_line (start 103.690582 52.983621) (end 103.693682 52.45352) (layer Edge.Cuts) (width 0.1))
 (gr_line (start 103.657662 53.37683) (end 103.690582 52.983621) (layer Edge.Cuts) (width 0.1))
 (gr_line (start 103.599622 53.698966) (end 103.657662 53.37683) (layer Edge.Cuts) (width 0.1))
 (gr_line (start 103.521142 54.01585) (end 103.599622 53.698966) (layer Edge.Cuts) (width 0.1))
 (gr_line (start 103.426902 54.3933) (end 103.521142 54.01585) (layer Edge.Cuts) (width 0.1))
 (gr_line (start 103.321583 54.89714) (end 103.426902 54.3933) (layer Edge.Cuts) (width 0.1))
 (gr_line (start 103.209871 55.59318) (end 103.321583 54.89714) (layer Edge.Cuts) (width 0.1))
 (gr_line (start 103.096452 56.54724) (end 103.209871 55.59318) (layer Edge.Cuts) (width 0.1))
 (segment (start 72.75 54.25) (end 72.75 55.25) (width 0.3) (layer B.Cu) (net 1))
 (segment (start 72.175 55.825) (end 71 55.825) (width 0.3) (layer F.Cu) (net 1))
 (segment (start 72.75 55.25) (end 72.175 55.825) (width 0.3) (layer F.Cu) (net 1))
 (via (at 72.75 55.25) (size 0.6) (drill 0.4) (layers F.Cu B.Cu) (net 1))
 (segment (start 80.25 52.5) (end 77.75 52.5) (width 0.3) (layer B.Cu) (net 1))
 (segment (start 89.25 52.5) (end 80.25 52.5) (width 0.3) (layer B.Cu) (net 1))
 (segment (start 76 54.25) (end 72.75 54.25) (width 0.3) (layer B.Cu) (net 1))
 (segment (start 72.75 54.25) (end 65.75 54.25) (width 0.3) (layer B.Cu) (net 1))
 (segment (start 77.75 52.5) (end 76 54.25) (width 0.3) (layer B.Cu) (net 1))
 (segment (start 65.75 54.25) (end 64 52.5) (width 0.3) (layer B.Cu) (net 1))
 (segment (start 64 52.5) (end 63.75 52.5) (width 0.3) (layer B.Cu) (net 1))
 (segment (start 70.75 48.925) (end 70.75 55.575) (width 0.3) (layer F.Cu) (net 1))
 (segment (start 91.75 45.25) (end 91.75 50) (width 0.3) (layer B.Cu) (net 1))
 (segment (start 89.25 52.5) (end 91.75 50) (width 0.3) (layer B.Cu) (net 1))
 (segment (start 91.75 45.25) (end 92.5 45.25) (width 0.3) (layer B.Cu) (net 1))
 (segment (start 96.75 45.25) (end 92.5 45.25) (width 0.3) (layer B.Cu) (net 1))
 (segment (start 91.75 45.25) (end 91.75 44.5) (width 0.3) (layer B.Cu) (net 1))
 (segment (start 91.75 40.5) (end 91.75 41.5) (width 0.3) (layer F.Cu) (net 1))
 (segment (start 91.75 44.5) (end 91.75 41.5) (width 0.3) (layer B.Cu) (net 1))
 (via (at 91.75 41.5) (size 0.6) (drill 0.4) (layers F.Cu B.Cu) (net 1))
 (segment (start 91.75 40.5) (end 91.35 40.1) (width 0.3) (layer F.Cu) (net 1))
 (segment (start 90 40.1) (end 91.35 40.1) (width 0.3) (layer F.Cu) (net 1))
 (segment (start 90.35 40.1) (end 90 40.1) (width 0.3) (layer F.Cu) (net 1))
 (segment (start 97.35 39.6) (end 97.5 39.75) (width 0.3) (layer F.Cu) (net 1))
 (segment (start 97.5 39.75) (end 97.5 41) (width 0.3) (layer F.Cu) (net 1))
 (segment (start 97.5 44.5) (end 96.75 45.25) (width 0.3) (layer B.Cu) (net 1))
 (segment (start 97.5 41) (end 97.5 44.5) (width 0.3) (layer B.Cu) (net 1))
 (via (at 97.5 41) (size 0.6) (drill 0.4) (layers F.Cu B.Cu) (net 1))
 (segment (start 97.35 39.6) (end 95.75 39.6) (width 0.3) (layer F.Cu) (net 1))
 (segment (start 95.75 39.6) (end 96.1 39.6) (width 0.3) (layer F.Cu) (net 1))
 (segment (start 95.75 46.75) (end 96 47) (width 0.3) (layer F.Cu) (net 2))
 (via (at 96 47) (size 0.6) (drill 0.4) (layers F.Cu B.Cu) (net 2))
 (segment (start 95.75 44.5) (end 95.75 46.75) (width 0.3) (layer F.Cu) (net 2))
 (segment (start 92.25 44.5) (end 95.75 44.5) (width 0.3) (layer F.Cu) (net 2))
 (segment (start 95.75 42.9) (end 95.75 44.5) (width 0.3) (layer F.Cu) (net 2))
 (segment (start 90 43.4) (end 90 45) (width 0.3) (layer F.Cu) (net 2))
 (segment (start 90 45) (end 88.75 46.25) (width 0.3) (layer F.Cu) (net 2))
 (segment (start 90 43.4) (end 91.15 43.4) (width 0.3) (layer F.Cu) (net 2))
 (segment (start 91.15 43.4) (end 92.25 44.5) (width 0.3) (layer F.Cu) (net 2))
 (segment (start 64.3 47.45) (end 64.3 49.175) (width 0.3) (layer F.Cu) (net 2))
 (segment (start 65.5 46.25) (end 64.3 47.45) (width 0.3) (layer F.Cu) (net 2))
 (segment (start 88.75 46.25) (end 65.5 46.25) (width 0.3) (layer F.Cu) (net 2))
 (segment (start 64.06 49.205) (end 64.06 50.19) (width 0.3) (layer F.Cu) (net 2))
 (segment (start 64.06 50.19) (end 62.75 51.5) (width 0.3) (layer F.Cu) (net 2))
 (segment (start 62.75 53.25) (end 64.05 54.55) (width 0.3) (layer F.Cu) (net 2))
 (segment (start 62.75 51.5) (end 62.75 53.25) (width 0.3) (layer F.Cu) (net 2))
 (segment (start 64.05 54.55) (end 64.05 55.575) (width 0.3) (layer F.Cu) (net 2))
 (segment (start 64.05 48.925) (end 64.05 49.95) (width 0.3) (layer F.Cu) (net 2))
 (segment (start 98.75 58.25) (end 98.75 57) (width 0.3) (layer B.Cu) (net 2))
 (segment (start 98.75 57) (end 100 55.75) (width 0.3) (layer B.Cu) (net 2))
 (segment (start 97.5 47) (end 96 47) (width 0.3) (layer B.Cu) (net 2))
 (segment (start 100 49.5) (end 97.5 47) (width 0.3) (layer B.Cu) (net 2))
 (segment (start 100 55.75) (end 100 49.5) (width 0.3) (layer B.Cu) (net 2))
 (segment (start 98.75 58.25) (end 98.75 59.75) (width 0.3) (layer B.Cu) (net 2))
 (segment (start 94.75 59.75) (end 95.5 60.5) (width 0.3) (layer B.Cu) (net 2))
 (segment (start 94.75 59.75) (end 94.75 58.25) (width 0.3) (layer B.Cu) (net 2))
 (segment (start 98 60.5) (end 95.5 60.5) (width 0.3) (layer B.Cu) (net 2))
 (segment (start 98.75 59.75) (end 98 60.5) (width 0.3) (layer B.Cu) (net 2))
 (segment (start 96 52.5) (end 96 54.75) (width 0.3) (layer B.Cu) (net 2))
 (segment (start 94.75 56) (end 94.75 58.25) (width 0.3) (layer B.Cu) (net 2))
 (segment (start 96 54.75) (end 94.75 56) (width 0.3) (layer B.Cu) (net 2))
 (segment (start 67.25 48.925) (end 67.25 55.575) (width 0.3) (layer F.Cu) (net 3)))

